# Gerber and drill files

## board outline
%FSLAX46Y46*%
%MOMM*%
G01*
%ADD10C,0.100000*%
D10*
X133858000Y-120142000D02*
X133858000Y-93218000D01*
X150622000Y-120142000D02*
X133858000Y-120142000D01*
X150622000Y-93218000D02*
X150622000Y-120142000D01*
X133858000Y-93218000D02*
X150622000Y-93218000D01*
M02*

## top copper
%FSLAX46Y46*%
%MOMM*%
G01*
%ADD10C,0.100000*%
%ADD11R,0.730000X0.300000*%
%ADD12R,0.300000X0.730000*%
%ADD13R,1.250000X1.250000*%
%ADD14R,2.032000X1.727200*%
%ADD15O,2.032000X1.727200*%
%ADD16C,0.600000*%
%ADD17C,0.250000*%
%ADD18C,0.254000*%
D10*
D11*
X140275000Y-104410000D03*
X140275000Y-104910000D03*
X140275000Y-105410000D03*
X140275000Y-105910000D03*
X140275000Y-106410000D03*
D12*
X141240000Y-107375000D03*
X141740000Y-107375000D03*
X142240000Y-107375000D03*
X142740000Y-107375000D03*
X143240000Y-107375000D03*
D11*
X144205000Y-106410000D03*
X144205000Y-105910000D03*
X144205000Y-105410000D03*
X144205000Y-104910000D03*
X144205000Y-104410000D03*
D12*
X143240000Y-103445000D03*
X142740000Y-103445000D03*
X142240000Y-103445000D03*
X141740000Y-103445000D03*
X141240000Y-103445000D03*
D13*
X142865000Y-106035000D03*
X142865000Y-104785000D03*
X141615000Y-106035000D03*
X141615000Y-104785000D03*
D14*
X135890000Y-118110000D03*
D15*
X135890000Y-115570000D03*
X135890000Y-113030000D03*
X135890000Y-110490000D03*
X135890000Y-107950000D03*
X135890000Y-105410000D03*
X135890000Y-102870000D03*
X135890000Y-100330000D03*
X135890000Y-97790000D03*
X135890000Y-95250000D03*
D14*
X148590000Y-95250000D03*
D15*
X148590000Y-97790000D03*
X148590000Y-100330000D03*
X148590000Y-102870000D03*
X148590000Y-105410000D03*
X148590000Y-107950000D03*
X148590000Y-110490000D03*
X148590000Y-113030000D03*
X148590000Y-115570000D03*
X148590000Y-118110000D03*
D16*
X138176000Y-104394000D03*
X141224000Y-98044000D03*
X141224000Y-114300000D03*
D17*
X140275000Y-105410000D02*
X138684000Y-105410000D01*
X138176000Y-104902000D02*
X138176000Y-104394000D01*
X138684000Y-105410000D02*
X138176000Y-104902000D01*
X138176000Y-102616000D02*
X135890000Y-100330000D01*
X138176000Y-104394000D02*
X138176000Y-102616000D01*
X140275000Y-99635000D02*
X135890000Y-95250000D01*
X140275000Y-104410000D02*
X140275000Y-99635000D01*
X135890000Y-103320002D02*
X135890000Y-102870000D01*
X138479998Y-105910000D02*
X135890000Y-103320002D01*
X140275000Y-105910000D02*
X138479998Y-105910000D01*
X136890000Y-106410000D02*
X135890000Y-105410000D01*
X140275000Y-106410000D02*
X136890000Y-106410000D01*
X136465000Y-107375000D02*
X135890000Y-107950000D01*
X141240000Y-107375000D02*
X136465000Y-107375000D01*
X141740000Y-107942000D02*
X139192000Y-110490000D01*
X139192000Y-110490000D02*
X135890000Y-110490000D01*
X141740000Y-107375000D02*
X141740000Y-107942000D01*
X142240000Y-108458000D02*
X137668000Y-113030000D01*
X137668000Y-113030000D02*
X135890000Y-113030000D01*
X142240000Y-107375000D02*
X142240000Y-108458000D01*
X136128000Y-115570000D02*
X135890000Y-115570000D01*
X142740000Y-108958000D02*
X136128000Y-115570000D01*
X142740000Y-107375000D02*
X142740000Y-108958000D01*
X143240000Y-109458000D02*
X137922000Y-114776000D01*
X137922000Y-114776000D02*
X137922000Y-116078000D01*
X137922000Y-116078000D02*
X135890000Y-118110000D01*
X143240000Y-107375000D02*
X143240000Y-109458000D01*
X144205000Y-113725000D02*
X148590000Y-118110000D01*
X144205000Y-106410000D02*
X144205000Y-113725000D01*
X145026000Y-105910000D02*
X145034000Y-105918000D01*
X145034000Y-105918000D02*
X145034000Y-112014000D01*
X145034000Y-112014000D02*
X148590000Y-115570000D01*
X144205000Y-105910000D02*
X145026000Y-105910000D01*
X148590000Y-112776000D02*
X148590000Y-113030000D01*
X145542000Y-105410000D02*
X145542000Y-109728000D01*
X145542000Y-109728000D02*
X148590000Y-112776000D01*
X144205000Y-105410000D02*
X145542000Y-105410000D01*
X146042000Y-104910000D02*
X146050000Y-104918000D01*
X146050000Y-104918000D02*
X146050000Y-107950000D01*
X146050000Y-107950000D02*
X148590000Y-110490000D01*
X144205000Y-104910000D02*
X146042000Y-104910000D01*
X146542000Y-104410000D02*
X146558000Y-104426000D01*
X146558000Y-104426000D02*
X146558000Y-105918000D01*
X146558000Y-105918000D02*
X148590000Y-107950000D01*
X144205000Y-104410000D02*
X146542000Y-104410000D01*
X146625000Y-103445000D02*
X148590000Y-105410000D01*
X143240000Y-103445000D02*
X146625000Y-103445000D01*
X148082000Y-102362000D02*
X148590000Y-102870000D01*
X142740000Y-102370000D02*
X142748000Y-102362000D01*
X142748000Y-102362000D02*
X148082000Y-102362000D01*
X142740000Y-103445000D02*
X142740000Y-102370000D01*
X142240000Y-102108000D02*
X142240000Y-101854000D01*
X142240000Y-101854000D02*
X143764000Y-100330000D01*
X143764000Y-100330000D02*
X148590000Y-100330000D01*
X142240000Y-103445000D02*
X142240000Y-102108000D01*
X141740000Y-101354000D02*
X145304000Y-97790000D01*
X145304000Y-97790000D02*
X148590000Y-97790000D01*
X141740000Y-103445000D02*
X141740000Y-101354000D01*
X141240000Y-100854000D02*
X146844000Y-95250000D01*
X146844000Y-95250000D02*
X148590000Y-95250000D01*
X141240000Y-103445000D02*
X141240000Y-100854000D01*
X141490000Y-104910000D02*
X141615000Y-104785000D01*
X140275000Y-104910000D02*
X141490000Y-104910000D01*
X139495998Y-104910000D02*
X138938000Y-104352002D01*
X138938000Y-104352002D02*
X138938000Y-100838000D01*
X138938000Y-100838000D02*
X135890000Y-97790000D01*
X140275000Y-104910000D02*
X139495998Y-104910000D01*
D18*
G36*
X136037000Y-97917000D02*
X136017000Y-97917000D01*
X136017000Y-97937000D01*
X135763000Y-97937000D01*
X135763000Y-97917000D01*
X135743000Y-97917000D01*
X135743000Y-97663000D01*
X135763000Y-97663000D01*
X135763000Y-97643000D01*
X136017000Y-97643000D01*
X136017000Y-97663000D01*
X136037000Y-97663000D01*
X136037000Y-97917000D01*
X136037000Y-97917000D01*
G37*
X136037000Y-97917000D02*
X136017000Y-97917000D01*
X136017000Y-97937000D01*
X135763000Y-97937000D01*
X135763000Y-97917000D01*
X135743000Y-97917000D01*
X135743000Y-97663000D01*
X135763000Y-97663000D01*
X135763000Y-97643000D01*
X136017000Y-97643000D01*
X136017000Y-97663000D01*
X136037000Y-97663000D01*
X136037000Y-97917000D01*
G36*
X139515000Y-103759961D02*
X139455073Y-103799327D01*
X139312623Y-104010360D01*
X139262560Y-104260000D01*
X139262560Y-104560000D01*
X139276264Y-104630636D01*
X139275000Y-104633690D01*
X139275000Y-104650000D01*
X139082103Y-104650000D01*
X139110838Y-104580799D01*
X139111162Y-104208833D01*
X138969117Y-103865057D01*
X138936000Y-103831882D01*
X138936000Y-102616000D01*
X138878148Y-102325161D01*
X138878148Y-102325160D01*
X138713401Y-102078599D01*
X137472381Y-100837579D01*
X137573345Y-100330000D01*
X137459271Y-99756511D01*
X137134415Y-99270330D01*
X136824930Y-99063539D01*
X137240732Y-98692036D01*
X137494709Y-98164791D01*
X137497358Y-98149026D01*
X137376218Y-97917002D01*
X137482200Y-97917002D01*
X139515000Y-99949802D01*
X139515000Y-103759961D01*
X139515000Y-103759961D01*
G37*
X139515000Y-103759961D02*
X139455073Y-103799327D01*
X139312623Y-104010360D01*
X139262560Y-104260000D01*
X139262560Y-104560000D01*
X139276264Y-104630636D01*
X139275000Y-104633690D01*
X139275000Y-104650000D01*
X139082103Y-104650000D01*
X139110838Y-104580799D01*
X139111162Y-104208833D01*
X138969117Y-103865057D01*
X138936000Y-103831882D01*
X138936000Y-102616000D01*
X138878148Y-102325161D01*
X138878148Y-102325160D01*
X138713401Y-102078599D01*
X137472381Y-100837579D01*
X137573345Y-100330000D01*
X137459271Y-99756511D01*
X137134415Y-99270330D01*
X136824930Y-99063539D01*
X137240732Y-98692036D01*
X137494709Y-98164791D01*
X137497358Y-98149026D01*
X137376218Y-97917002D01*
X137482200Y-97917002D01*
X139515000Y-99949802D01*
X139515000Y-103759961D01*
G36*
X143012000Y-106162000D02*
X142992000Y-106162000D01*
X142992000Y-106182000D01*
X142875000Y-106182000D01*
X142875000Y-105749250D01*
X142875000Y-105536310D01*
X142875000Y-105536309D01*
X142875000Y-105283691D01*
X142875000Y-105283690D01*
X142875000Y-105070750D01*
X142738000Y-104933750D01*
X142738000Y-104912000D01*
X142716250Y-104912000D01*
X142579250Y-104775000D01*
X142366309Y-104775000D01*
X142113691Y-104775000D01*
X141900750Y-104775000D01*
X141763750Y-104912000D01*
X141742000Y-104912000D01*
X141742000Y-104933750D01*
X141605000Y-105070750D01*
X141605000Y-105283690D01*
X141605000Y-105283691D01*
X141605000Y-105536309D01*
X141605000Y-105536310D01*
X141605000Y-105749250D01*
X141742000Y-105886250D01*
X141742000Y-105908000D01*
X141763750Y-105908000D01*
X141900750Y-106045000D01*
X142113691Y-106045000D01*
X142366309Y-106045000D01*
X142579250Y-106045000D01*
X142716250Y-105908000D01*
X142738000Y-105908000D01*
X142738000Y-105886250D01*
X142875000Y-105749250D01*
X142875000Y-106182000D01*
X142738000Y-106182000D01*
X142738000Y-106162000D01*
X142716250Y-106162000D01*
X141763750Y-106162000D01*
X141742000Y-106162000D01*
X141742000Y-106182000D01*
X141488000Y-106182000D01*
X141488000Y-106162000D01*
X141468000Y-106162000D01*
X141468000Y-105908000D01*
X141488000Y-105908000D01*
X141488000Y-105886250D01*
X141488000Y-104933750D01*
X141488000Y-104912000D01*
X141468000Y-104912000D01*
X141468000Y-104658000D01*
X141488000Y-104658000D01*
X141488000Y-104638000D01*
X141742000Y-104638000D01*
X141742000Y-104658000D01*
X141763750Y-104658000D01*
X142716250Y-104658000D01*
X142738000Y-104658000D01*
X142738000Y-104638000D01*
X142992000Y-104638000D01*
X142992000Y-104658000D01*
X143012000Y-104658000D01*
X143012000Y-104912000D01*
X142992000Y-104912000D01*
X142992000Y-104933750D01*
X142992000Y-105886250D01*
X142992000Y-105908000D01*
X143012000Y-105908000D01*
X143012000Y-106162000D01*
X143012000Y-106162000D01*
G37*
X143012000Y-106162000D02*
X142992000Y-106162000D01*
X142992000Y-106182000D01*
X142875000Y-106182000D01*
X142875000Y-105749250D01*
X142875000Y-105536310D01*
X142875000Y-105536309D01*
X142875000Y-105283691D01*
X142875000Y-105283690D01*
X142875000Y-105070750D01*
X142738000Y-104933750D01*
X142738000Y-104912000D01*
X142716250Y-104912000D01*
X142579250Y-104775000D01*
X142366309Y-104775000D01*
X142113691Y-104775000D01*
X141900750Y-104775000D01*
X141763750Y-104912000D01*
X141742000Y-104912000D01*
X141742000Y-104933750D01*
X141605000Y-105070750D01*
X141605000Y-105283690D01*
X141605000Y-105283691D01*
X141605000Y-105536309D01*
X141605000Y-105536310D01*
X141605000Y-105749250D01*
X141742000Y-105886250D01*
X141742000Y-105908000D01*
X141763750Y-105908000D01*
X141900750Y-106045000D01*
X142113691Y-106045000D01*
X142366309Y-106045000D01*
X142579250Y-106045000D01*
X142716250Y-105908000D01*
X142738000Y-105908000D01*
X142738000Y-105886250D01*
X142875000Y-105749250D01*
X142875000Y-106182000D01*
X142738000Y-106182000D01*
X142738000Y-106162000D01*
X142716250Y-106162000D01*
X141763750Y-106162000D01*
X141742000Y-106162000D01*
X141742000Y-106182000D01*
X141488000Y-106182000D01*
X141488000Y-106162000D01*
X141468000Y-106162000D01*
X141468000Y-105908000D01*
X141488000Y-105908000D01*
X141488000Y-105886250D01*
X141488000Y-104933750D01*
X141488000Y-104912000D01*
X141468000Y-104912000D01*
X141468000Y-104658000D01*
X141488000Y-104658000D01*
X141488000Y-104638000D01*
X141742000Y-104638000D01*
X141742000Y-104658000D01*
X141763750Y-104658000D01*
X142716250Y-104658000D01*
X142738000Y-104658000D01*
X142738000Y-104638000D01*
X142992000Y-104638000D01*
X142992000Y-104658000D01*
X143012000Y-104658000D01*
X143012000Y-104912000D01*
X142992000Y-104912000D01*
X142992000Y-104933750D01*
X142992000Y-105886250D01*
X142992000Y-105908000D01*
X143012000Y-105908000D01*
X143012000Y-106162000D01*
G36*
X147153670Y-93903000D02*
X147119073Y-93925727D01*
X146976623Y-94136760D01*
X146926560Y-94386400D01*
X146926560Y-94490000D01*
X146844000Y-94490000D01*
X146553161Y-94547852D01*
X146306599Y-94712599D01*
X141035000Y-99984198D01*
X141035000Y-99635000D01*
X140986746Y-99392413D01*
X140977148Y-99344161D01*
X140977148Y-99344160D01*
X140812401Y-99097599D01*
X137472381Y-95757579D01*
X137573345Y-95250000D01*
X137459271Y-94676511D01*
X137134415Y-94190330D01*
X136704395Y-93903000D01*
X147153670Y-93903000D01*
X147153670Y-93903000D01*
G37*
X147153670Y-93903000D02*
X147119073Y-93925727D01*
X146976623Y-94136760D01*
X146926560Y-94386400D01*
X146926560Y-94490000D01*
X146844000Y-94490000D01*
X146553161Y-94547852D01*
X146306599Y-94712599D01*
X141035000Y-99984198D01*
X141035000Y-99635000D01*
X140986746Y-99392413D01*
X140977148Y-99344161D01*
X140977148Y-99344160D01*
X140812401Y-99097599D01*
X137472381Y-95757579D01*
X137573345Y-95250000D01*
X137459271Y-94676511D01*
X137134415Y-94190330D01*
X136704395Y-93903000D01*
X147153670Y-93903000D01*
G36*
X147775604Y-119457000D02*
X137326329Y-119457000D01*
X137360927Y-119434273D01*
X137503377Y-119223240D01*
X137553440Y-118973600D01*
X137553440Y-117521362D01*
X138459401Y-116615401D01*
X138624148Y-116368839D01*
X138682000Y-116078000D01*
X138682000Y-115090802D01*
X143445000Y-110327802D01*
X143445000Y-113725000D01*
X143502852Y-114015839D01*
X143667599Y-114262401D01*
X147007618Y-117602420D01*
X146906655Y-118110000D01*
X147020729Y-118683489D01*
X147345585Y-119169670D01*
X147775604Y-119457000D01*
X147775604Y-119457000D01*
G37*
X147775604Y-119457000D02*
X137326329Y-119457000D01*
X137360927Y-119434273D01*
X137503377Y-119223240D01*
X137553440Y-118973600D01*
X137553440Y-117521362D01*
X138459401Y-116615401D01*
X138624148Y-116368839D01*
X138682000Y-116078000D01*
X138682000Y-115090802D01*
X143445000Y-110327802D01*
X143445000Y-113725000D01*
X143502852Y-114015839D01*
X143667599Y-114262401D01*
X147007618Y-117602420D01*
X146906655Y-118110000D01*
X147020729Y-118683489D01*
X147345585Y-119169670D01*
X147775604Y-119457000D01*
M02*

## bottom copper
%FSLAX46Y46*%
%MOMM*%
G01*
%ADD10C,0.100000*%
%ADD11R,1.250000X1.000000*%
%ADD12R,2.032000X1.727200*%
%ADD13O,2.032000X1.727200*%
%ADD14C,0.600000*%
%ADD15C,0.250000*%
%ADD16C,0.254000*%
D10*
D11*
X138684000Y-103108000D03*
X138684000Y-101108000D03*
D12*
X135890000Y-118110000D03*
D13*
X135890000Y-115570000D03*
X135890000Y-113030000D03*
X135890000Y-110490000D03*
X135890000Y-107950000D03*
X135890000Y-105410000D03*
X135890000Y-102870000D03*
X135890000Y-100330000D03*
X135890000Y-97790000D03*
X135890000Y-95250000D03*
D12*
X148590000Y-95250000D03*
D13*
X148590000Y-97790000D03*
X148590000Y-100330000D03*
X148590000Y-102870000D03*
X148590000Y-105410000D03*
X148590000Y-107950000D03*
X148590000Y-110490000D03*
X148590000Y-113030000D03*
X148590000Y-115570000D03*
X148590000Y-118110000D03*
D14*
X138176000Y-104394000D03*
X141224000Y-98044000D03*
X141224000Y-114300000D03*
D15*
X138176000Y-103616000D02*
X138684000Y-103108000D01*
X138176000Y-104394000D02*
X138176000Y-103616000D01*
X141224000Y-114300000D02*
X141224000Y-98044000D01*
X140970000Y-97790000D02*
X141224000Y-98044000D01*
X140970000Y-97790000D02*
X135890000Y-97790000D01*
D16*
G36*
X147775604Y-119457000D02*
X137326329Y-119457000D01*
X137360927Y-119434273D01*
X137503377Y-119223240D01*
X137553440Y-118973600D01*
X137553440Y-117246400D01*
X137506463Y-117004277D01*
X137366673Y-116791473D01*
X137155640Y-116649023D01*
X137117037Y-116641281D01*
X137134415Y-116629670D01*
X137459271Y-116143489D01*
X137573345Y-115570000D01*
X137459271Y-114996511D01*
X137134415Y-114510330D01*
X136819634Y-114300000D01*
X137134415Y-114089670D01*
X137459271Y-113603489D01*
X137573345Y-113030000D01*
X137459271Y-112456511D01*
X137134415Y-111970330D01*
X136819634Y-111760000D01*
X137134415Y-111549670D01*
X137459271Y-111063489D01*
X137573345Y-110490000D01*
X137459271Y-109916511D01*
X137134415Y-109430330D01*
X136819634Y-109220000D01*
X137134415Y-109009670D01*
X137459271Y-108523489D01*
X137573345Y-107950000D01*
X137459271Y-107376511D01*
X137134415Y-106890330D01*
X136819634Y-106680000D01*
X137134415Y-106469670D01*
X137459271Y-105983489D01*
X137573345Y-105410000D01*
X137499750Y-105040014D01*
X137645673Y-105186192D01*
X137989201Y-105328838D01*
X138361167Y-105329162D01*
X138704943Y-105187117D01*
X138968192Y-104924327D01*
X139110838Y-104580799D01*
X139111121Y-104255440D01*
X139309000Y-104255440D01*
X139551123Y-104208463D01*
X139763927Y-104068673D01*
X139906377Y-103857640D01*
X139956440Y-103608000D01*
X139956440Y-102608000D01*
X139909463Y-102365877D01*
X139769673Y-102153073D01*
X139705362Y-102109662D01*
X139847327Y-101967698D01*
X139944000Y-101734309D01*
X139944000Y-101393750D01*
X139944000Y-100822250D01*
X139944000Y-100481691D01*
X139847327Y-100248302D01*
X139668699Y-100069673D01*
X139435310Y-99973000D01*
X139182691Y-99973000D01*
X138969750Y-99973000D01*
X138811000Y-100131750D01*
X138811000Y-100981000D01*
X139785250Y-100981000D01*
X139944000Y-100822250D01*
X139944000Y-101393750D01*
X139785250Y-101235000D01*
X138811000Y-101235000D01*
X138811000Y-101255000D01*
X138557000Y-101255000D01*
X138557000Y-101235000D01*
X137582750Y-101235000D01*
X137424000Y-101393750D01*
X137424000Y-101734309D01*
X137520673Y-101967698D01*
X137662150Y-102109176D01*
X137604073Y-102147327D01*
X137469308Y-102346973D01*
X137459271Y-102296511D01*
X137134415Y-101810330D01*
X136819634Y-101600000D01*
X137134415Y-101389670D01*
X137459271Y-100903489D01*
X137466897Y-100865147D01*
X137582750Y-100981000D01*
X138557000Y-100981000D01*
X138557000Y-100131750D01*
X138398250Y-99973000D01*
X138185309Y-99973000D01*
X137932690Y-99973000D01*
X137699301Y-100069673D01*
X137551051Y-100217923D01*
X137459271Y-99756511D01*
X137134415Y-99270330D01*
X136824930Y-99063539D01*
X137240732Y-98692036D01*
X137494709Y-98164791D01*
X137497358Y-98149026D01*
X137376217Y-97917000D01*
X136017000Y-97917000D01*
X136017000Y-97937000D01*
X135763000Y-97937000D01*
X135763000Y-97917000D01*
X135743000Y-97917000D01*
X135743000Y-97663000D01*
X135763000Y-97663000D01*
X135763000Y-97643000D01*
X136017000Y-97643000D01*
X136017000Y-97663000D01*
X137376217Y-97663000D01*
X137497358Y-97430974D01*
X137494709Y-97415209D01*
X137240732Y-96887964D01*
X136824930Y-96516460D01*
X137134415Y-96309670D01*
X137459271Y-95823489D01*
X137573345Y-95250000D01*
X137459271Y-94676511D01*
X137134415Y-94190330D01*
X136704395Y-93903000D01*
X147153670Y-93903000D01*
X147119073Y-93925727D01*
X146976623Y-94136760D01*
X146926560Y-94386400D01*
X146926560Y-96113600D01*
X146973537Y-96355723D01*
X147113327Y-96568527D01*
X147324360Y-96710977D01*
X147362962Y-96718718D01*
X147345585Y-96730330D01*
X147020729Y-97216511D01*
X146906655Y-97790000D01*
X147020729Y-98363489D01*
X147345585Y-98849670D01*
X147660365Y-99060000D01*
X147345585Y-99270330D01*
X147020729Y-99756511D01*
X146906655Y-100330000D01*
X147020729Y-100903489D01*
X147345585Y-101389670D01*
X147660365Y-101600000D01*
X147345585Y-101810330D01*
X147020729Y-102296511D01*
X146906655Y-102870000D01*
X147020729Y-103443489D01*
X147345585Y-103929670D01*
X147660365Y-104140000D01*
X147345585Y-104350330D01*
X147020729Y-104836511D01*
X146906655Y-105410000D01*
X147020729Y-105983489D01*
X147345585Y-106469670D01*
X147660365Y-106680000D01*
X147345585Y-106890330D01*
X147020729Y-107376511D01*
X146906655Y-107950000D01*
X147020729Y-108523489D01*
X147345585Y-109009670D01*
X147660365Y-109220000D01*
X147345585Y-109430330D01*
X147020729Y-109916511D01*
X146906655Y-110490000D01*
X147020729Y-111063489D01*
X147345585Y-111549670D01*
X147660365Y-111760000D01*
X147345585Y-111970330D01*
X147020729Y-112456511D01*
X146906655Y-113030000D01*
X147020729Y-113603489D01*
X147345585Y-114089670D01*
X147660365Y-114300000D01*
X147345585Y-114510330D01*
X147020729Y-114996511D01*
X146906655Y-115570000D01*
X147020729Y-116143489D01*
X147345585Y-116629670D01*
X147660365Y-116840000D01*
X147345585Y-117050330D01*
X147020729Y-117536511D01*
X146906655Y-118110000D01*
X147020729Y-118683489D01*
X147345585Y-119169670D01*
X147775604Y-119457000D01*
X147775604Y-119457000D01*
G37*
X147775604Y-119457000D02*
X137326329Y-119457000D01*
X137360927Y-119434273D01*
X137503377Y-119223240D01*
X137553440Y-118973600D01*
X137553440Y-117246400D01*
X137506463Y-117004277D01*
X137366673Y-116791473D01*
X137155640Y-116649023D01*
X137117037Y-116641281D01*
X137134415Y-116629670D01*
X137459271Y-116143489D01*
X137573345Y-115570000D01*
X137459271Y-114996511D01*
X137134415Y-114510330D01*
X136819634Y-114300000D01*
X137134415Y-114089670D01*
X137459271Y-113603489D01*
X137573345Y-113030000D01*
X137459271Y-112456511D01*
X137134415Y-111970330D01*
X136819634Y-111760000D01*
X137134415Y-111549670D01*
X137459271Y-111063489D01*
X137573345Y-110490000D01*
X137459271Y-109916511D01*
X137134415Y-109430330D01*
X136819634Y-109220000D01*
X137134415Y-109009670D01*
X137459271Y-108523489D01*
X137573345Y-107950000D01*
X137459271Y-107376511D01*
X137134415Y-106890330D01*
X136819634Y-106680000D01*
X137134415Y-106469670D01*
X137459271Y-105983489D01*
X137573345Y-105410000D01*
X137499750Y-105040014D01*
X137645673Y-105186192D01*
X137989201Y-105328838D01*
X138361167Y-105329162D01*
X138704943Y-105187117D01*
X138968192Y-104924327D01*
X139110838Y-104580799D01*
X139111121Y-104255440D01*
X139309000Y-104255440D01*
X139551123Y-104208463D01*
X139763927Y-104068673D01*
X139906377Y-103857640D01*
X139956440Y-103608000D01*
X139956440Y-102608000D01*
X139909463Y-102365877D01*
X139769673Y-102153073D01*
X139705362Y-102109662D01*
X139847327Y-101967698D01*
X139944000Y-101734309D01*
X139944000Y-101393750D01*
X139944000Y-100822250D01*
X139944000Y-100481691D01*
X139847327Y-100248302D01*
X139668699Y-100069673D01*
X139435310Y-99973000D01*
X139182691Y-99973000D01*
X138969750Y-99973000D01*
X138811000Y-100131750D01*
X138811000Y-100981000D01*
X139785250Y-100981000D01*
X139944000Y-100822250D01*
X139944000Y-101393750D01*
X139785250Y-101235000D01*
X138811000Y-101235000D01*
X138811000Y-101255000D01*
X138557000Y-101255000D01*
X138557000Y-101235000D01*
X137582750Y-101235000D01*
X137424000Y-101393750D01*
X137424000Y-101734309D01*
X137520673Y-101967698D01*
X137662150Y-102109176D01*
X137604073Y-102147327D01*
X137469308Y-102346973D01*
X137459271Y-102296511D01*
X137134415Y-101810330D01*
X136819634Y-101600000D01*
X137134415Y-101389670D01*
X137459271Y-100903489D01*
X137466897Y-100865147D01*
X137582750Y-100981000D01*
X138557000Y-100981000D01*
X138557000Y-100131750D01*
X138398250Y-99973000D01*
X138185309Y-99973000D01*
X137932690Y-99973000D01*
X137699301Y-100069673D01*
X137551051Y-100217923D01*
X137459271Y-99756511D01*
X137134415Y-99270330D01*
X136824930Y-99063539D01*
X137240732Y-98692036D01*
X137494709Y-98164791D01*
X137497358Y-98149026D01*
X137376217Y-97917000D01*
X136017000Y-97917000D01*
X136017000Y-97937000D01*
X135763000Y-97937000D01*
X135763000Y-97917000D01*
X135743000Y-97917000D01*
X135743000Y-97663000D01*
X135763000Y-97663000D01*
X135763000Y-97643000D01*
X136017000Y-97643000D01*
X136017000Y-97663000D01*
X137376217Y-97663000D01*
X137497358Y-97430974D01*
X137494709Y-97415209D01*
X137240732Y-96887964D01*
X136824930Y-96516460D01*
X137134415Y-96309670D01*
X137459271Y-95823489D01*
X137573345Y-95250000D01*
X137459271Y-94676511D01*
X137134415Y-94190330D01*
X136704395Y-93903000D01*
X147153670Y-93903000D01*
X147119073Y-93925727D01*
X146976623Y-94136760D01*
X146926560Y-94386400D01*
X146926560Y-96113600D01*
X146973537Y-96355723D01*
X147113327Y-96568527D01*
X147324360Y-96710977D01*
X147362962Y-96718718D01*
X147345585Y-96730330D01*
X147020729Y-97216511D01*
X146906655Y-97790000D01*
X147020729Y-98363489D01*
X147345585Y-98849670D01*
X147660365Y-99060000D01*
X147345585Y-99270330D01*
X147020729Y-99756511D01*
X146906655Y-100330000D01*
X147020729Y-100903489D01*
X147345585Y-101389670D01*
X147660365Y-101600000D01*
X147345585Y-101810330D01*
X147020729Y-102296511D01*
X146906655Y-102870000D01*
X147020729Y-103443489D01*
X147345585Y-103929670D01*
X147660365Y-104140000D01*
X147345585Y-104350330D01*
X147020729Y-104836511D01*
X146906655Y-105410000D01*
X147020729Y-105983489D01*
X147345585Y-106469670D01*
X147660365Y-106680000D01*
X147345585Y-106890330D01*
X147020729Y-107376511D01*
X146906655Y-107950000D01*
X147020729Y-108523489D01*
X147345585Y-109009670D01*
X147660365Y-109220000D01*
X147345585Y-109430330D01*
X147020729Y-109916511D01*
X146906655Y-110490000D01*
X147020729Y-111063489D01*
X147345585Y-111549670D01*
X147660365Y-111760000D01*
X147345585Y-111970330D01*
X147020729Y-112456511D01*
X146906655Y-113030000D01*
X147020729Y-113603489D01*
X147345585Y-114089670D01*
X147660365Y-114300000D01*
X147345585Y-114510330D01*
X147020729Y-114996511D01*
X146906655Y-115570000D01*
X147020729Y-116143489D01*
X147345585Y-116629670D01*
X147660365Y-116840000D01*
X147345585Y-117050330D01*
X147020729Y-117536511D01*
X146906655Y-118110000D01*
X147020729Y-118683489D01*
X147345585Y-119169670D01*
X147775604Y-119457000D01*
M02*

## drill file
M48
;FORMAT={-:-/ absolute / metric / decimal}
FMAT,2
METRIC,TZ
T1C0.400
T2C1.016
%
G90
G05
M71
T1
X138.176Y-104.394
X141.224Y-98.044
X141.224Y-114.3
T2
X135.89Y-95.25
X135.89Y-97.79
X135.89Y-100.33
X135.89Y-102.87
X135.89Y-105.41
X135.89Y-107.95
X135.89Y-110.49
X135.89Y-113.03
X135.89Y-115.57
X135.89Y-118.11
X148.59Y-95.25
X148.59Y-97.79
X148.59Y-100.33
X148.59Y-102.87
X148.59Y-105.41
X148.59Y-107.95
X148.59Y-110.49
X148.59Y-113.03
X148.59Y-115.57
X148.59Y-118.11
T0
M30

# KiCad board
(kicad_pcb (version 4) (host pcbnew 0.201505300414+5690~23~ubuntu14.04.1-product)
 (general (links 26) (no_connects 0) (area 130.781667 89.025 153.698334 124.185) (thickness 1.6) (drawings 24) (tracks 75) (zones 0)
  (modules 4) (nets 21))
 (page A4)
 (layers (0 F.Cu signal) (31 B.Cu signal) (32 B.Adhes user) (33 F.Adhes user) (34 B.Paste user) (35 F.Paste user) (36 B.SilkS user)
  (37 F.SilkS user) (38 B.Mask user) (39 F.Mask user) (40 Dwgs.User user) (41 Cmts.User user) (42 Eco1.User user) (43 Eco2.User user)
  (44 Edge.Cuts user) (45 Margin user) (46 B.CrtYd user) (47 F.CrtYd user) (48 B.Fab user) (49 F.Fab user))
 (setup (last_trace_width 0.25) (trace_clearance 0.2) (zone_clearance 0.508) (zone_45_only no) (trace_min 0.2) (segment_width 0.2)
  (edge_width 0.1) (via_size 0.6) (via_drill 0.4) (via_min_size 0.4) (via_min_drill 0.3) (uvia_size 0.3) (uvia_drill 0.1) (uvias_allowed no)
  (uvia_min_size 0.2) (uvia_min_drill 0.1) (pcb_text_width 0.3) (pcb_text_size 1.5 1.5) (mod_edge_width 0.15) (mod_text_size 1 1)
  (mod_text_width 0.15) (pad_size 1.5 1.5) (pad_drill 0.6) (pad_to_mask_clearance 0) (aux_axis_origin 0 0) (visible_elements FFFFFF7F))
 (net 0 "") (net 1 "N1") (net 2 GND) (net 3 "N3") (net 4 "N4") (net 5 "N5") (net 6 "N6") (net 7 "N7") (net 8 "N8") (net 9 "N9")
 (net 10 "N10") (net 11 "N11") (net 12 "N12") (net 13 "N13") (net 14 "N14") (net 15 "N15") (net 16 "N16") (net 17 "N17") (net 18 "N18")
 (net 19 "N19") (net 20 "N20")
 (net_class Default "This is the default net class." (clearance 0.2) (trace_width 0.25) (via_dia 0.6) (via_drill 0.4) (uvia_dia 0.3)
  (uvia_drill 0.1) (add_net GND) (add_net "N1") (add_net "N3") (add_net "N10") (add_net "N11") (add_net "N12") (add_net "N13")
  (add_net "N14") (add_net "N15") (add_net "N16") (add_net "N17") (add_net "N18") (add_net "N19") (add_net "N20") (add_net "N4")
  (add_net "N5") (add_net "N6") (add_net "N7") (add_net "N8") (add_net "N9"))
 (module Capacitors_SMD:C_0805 (layer B.Cu) (at 138.684 102.108 90)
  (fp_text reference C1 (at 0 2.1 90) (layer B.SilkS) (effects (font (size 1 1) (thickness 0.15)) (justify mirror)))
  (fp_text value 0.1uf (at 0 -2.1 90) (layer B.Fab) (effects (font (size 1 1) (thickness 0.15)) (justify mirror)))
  (pad 1 smd rect (at -1 0 90) (size 1 1.25) (layers B.Cu B.Paste B.Mask) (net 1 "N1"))
  (pad 2 smd rect (at 1 0 90) (size 1 1.25) (layers B.Cu B.Paste B.Mask) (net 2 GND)))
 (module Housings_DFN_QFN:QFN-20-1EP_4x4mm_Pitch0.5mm (layer F.Cu) (at 142.24 105.41)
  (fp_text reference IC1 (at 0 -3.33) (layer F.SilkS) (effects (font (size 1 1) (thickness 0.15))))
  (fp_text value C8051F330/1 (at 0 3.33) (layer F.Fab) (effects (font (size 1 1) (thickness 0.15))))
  (pad 1 smd rect (at -1.965 -1) (size 0.73 0.3) (layers F.Cu F.Paste F.Mask) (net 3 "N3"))
  (pad 2 smd rect (at -1.965 -0.5) (size 0.73 0.3) (layers F.Cu F.Paste F.Mask) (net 2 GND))
  (pad 3 smd rect (at -1.965 0) (size 0.73 0.3) (layers F.Cu F.Paste F.Mask) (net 1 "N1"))
  (pad 4 smd rect (at -1.965 0.5) (size 0.73 0.3) (layers F.Cu F.Paste F.Mask) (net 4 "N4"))
  (pad 5 smd rect (at -1.965 1) (size 0.73 0.3) (layers F.Cu F.Paste F.Mask) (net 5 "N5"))
  (pad 6 smd rect (at -1 1.965 90) (size 0.73 0.3) (layers F.Cu F.Paste F.Mask) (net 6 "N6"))
  (pad 7 smd rect (at -0.5 1.965 90) (size 0.73 0.3) (layers F.Cu F.Paste F.Mask) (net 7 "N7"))
  (pad 8 smd rect (at 0 1.965 90) (size 0.73 0.3) (layers F.Cu F.Paste F.Mask) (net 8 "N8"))
  (pad 9 smd rect (at 0.5 1.965 90) (size 0.73 0.3) (layers F.Cu F.Paste F.Mask) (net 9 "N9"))
  (pad 10 smd rect (at 1 1.965 90) (size 0.73 0.3) (layers F.Cu F.Paste F.Mask) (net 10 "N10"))
  (pad 11 smd rect (at 1.965 1) (size 0.73 0.3) (layers F.Cu F.Paste F.Mask) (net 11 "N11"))
  (pad 12 smd rect (at 1.965 0.5) (size 0.73 0.3) (layers F.Cu F.Paste F.Mask) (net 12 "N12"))
  (pad 13 smd rect (at 1.965 0) (size 0.73 0.3) (layers F.Cu F.Paste F.Mask) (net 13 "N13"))
  (pad 14 smd rect (at 1.965 -0.5) (size 0.73 0.3) (layers F.Cu F.Paste F.Mask) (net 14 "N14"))
  (pad 15 smd rect (at 1.965 -1) (size 0.73 0.3) (layers F.Cu F.Paste F.Mask) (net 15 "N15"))
  (pad 16 smd rect (at 1 -1.965 90) (size 0.73 0.3) (layers F.Cu F.Paste F.Mask) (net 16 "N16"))
  (pad 17 smd rect (at 0.5 -1.965 90) (size 0.73 0.3) (layers F.Cu F.Paste F.Mask) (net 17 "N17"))
  (pad 18 smd rect (at 0 -1.965 90) (size 0.73 0.3) (layers F.Cu F.Paste F.Mask) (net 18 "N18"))
  (pad 19 smd rect (at -0.5 -1.965 90) (size 0.73 0.3) (layers F.Cu F.Paste F.Mask) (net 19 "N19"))
  (pad 20 smd rect (at -1 -1.965 90) (size 0.73 0.3) (layers F.Cu F.Paste F.Mask) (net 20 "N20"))
  (pad 21 smd rect (at 0.625 0.625) (size 1.25 1.25) (layers F.Cu F.Paste F.Mask) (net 2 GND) (solder_paste_margin_ratio -0.2))
  (pad 21 smd rect (at 0.625 -0.625) (size 1.25 1.25) (layers F.Cu F.Paste F.Mask) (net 2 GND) (solder_paste_margin_ratio -0.2))
  (pad 21 smd rect (at -0.625 0.625) (size 1.25 1.25) (layers F.Cu F.Paste F.Mask) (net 2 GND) (solder_paste_margin_ratio -0.2))
  (pad 21 smd rect (at -0.625 -0.625) (size 1.25 1.25) (layers F.Cu F.Paste F.Mask) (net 2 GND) (solder_paste_margin_ratio -0.2)))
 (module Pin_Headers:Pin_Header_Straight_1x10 (layer F.Cu) (at 135.89 118.11 180)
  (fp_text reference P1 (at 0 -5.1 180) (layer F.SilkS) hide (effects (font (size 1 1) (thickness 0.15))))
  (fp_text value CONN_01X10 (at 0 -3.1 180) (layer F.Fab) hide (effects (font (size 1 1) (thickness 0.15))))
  (pad 1 thru_hole rect (at 0 0 180) (size 2.032 1.7272) (drill 1.016) (layers *.Cu *.Mask F.SilkS) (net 10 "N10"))
  (pad 2 thru_hole oval (at 0 2.54 180) (size 2.032 1.7272) (drill 1.016) (layers *.Cu *.Mask F.SilkS) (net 9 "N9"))
  (pad 3 thru_hole oval (at 0 5.08 180) (size 2.032 1.7272) (drill 1.016) (layers *.Cu *.Mask F.SilkS) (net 8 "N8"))
  (pad 4 thru_hole oval (at 0 7.62 180) (size 2.032 1.7272) (drill 1.016) (layers *.Cu *.Mask F.SilkS) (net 7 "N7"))
  (pad 5 thru_hole oval (at 0 10.16 180) (size 2.032 1.7272) (drill 1.016) (layers *.Cu *.Mask F.SilkS) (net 6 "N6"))
  (pad 6 thru_hole oval (at 0 12.7 180) (size 2.032 1.7272) (drill 1.016) (layers *.Cu *.Mask F.SilkS) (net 5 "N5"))
  (pad 7 thru_hole oval (at 0 15.24 180) (size 2.032 1.7272) (drill 1.016) (layers *.Cu *.Mask F.SilkS) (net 4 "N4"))
  (pad 8 thru_hole oval (at 0 17.78 180) (size 2.032 1.7272) (drill 1.016) (layers *.Cu *.Mask F.SilkS) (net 1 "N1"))
  (pad 9 thru_hole oval (at 0 20.32 180) (size 2.032 1.7272) (drill 1.016) (layers *.Cu *.Mask F.SilkS) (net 2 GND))
  (pad 10 thru_hole oval (at 0 22.86 180) (size 2.032 1.7272) (drill 1.016) (layers *.Cu *.Mask F.SilkS) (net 3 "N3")))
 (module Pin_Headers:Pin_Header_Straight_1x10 (layer F.Cu) (at 148.59 95.25)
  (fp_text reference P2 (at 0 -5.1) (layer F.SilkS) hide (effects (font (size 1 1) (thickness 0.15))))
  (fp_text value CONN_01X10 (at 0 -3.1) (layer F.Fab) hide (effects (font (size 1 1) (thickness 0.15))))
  (pad 1 thru_hole rect (at 0 0) (size 2.032 1.7272) (drill 1.016) (layers *.Cu *.Mask F.SilkS) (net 20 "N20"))
  (pad 2 thru_hole oval (at 0 2.54) (size 2.032 1.7272) (drill 1.016) (layers *.Cu *.Mask F.SilkS) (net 19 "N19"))
  (pad 3 thru_hole oval (at 0 5.08) (size 2.032 1.7272) (drill 1.016) (layers *.Cu *.Mask F.SilkS) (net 18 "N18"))
  (pad 4 thru_hole oval (at 0 7.62) (size 2.032 1.7272) (drill 1.016) (layers *.Cu *.Mask F.SilkS) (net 17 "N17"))
  (pad 5 thru_hole oval (at 0 10.16) (size 2.032 1.7272) (drill 1.016) (layers *.Cu *.Mask F.SilkS) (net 16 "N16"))
  (pad 6 thru_hole oval (at 0 12.7) (size 2.032 1.7272) (drill 1.016) (layers *.Cu *.Mask F.SilkS) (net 15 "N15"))
  (pad 7 thru_hole oval (at 0 15.24) (size 2.032 1.7272) (drill 1.016) (layers *.Cu *.Mask F.SilkS) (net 14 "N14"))
  (pad 8 thru_hole oval (at 0 17.78) (size 2.032 1.7272) (drill 1.016) (layers *.Cu *.Mask F.SilkS) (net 13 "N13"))
  (pad 9 thru_hole oval (at 0 20.32) (size 2.032 1.7272) (drill 1.016) (layers *.Cu *.Mask F.SilkS) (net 12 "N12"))
  (pad 10 thru_hole oval (at 0 22.86) (size 2.032 1.7272) (drill 1.016) (layers *.Cu *.Mask F.SilkS) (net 11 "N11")))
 (gr_line (start 133.858 120.142) (end 133.858 93.218) (angle 90) (layer Edge.Cuts) (width 0.1))
 (gr_line (start 150.622 120.142) (end 133.858 120.142) (angle 90) (layer Edge.Cuts) (width 0.1))
 (gr_line (start 150.622 93.218) (end 150.622 120.142) (angle 90) (layer Edge.Cuts) (width 0.1))
 (gr_line (start 133.858 93.218) (end 150.622 93.218) (angle 90) (layer Edge.Cuts) (width 0.1))
 (segment (start 138.176 103.616) (end 138.684 103.108) (width 0.25) (layer B.Cu) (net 1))
 (segment (start 140.275 105.41) (end 138.684 105.41) (width 0.25) (layer F.Cu) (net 1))
 (via (at 138.176 104.394) (size 0.6) (drill 0.4) (layers F.Cu B.Cu) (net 1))
 (segment (start 138.176 104.902) (end 138.176 104.394) (width 0.25) (layer F.Cu) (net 1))
 (segment (start 138.684 105.41) (end 138.176 104.902) (width 0.25) (layer F.Cu) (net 1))
 (segment (start 138.176 104.394) (end 138.176 103.616) (width 0.25) (layer B.Cu) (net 1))
 (segment (start 138.176 102.616) (end 135.89 100.33) (width 0.25) (layer F.Cu) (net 1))
 (segment (start 138.176 104.394) (end 138.176 102.616) (width 0.25) (layer F.Cu) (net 1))
 (segment (start 140.275 99.635) (end 135.89 95.25) (width 0.25) (layer F.Cu) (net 3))
 (segment (start 140.275 104.41) (end 140.275 99.635) (width 0.25) (layer F.Cu) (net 3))
 (segment (start 135.89 103.320002) (end 135.89 102.87) (width 0.25) (layer F.Cu) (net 4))
 (segment (start 138.479998 105.91) (end 135.89 103.320002) (width 0.25) (layer F.Cu) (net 4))
 (segment (start 140.275 105.91) (end 138.479998 105.91) (width 0.25) (layer F.Cu) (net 4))
 (segment (start 136.89 106.41) (end 135.89 105.41) (width 0.25) (layer F.Cu) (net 5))
 (segment (start 140.275 106.41) (end 136.89 106.41) (width 0.25) (layer F.Cu) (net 5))
 (segment (start 136.465 107.375) (end 135.89 107.95) (width 0.25) (layer F.Cu) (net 6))
 (segment (start 141.24 107.375) (end 136.465 107.375) (width 0.25) (layer F.Cu) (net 6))
 (segment (start 141.74 107.942) (end 139.192 110.49) (width 0.25) (layer F.Cu) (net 7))
 (segment (start 139.192 110.49) (end 135.89 110.49) (width 0.25) (layer F.Cu) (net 7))
 (segment (start 141.74 107.375) (end 141.74 107.942) (width 0.25) (layer F.Cu) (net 7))
 (segment (start 142.24 108.458) (end 137.668 113.03) (width 0.25) (layer F.Cu) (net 8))
 (segment (start 137.668 113.03) (end 135.89 113.03) (width 0.25) (layer F.Cu) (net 8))
 (segment (start 142.24 107.375) (end 142.24 108.458) (width 0.25) (layer F.Cu) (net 8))
 (segment (start 136.128 115.57) (end 135.89 115.57) (width 0.25) (layer F.Cu) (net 9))
 (segment (start 142.74 108.958) (end 136.128 115.57) (width 0.25) (layer F.Cu) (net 9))
 (segment (start 142.74 107.375) (end 142.74 108.958) (width 0.25) (layer F.Cu) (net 9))
 (segment (start 143.24 109.458) (end 137.922 114.776) (width 0.25) (layer F.Cu) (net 10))
 (segment (start 137.922 114.776) (end 137.922 116.078) (width 0.25) (layer F.Cu) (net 10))
 (segment (start 137.922 116.078) (end 135.89 118.11) (width 0.25) (layer F.Cu) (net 10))
 (segment (start 143.24 107.375) (end 143.24 109.458) (width 0.25) (layer F.Cu) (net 10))
 (segment (start 144.205 113.725) (end 148.59 118.11) (width 0.25) (layer F.Cu) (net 11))
 (segment (start 144.205 106.41) (end 144.205 113.725) (width 0.25) (layer F.Cu) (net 11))
 (segment (start 145.026 105.91) (end 145.034 105.918) (width 0.25) (layer F.Cu) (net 12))
 (segment (start 145.034 105.918) (end 145.034 112.014) (width 0.25) (layer F.Cu) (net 12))
 (segment (start 145.034 112.014) (end 148.59 115.57) (width 0.25) (layer F.Cu) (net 12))
 (segment (start 144.205 105.91) (end 145.026 105.91) (width 0.25) (layer F.Cu) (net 12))
 (segment (start 148.59 112.776) (end 148.59 113.03) (width 0.25) (layer F.Cu) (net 13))
 (segment (start 145.542 105.41) (end 145.542 109.728) (width 0.25) (layer F.Cu) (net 13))
 (segment (start 145.542 109.728) (end 148.59 112.776) (width 0.25) (layer F.Cu) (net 13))
 (segment (start 144.205 105.41) (end 145.542 105.41) (width 0.25) (layer F.Cu) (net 13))
 (segment (start 146.042 104.91) (end 146.05 104.918) (width 0.25) (layer F.Cu) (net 14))
 (segment (start 146.05 104.918) (end 146.05 107.95) (width 0.25) (layer F.Cu) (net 14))
 (segment (start 146.05 107.95) (end 148.59 110.49) (width 0.25) (layer F.Cu) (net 14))
 (segment (start 144.205 104.91) (end 146.042 104.91) (width 0.25) (layer F.Cu) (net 14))
 (segment (start 146.542 104.41) (end 146.558 104.426) (width 0.25) (layer F.Cu) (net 15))
 (segment (start 146.558 104.426) (end 146.558 105.918) (width 0.25) (layer F.Cu) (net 15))
 (segment (start 146.558 105.918) (end 148.59 107.95) (width 0.25) (layer F.Cu) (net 15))
 (segment (start 144.205 104.41) (end 146.542 104.41) (width 0.25) (layer F.Cu) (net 15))
 (segment (start 146.625 103.445) (end 148.59 105.41) (width 0.25) (layer F.Cu) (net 16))
 (segment (start 143.24 103.445) (end 146.625 103.445) (width 0.25) (layer F.Cu) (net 16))
 (segment (start 148.082 102.362) (end 148.59 102.87) (width 0.25) (layer F.Cu) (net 17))
 (segment (start 142.74 102.37) (end 142.748 102.362) (width 0.25) (layer F.Cu) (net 17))
 (segment (start 142.748 102.362) (end 148.082 102.362) (width 0.25) (layer F.Cu) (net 17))
 (segment (start 142.74 103.445) (end 142.74 102.37) (width 0.25) (layer F.Cu) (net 17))
 (segment (start 142.24 102.108) (end 142.24 101.854) (width 0.25) (layer F.Cu) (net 18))
 (segment (start 142.24 101.854) (end 143.764 100.33) (width 0.25) (layer F.Cu) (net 18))
 (segment (start 143.764 100.33) (end 148.59 100.33) (width 0.25) (layer F.Cu) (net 18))
 (segment (start 142.24 103.445) (end 142.24 102.108) (width 0.25) (layer F.Cu) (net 18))
 (segment (start 141.74 101.354) (end 145.304 97.79) (width 0.25) (layer F.Cu) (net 19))
 (segment (start 145.304 97.79) (end 148.59 97.79) (width 0.25) (layer F.Cu) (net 19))
 (segment (start 141.74 103.445) (end 141.74 101.354) (width 0.25) (layer F.Cu) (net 19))
 (segment (start 141.24 100.854) (end 146.844 95.25) (width 0.25) (layer F.Cu) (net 20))
 (segment (start 146.844 95.25) (end 148.59 95.25) (width 0.25) (layer F.Cu) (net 20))
 (segment (start 141.24 103.445) (end 141.24 100.854) (width 0.25) (layer F.Cu) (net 20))
 (segment (start 141.224 114.3) (end 141.224 98.044) (width 0.25) (layer B.Cu) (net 2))
 (segment (start 140.97 97.79) (end 141.224 98.044) (width 0.25) (layer B.Cu) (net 2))
 (via (at 141.224 98.044) (size 0.6) (layers F.Cu B.Cu) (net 2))
 (segment (start 140.97 97.79) (end 135.89 97.79) (width 0.25) (layer B.Cu) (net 2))
 (via (at 141.224 114.3) (size 0.6) (layers F.Cu B.Cu) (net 2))
 (segment (start 141.49 104.91) (end 141.615 104.785) (width 0.25) (layer F.Cu) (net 2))
 (segment (start 140.275 104.91) (end 141.49 104.91) (width 0.25) (layer F.Cu) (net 2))
 (segment (start 139.495998 104.91) (end 138.938 104.352002) (width 0.25) (layer F.Cu) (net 2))
 (segment (start 138.938 104.352002) (end 138.938 100.838) (width 0.25) (layer F.Cu) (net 2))
 (segment (start 138.938 100.838) (end 135.89 97.79) (width 0.25) (layer F.Cu) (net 2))
 (segment (start 140.275 104.91) (end 139.495998 104.91) (width 0.25) (layer F.Cu) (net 2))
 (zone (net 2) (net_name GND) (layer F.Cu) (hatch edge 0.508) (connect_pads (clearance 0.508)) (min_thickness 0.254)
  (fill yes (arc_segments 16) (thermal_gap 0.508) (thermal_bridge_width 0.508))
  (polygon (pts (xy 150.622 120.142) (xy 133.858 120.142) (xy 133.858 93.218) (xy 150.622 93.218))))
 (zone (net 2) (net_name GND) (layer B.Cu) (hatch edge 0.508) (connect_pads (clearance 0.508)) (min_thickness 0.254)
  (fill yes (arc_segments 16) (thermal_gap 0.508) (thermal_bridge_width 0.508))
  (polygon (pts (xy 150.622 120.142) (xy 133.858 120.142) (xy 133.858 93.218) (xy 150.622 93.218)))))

